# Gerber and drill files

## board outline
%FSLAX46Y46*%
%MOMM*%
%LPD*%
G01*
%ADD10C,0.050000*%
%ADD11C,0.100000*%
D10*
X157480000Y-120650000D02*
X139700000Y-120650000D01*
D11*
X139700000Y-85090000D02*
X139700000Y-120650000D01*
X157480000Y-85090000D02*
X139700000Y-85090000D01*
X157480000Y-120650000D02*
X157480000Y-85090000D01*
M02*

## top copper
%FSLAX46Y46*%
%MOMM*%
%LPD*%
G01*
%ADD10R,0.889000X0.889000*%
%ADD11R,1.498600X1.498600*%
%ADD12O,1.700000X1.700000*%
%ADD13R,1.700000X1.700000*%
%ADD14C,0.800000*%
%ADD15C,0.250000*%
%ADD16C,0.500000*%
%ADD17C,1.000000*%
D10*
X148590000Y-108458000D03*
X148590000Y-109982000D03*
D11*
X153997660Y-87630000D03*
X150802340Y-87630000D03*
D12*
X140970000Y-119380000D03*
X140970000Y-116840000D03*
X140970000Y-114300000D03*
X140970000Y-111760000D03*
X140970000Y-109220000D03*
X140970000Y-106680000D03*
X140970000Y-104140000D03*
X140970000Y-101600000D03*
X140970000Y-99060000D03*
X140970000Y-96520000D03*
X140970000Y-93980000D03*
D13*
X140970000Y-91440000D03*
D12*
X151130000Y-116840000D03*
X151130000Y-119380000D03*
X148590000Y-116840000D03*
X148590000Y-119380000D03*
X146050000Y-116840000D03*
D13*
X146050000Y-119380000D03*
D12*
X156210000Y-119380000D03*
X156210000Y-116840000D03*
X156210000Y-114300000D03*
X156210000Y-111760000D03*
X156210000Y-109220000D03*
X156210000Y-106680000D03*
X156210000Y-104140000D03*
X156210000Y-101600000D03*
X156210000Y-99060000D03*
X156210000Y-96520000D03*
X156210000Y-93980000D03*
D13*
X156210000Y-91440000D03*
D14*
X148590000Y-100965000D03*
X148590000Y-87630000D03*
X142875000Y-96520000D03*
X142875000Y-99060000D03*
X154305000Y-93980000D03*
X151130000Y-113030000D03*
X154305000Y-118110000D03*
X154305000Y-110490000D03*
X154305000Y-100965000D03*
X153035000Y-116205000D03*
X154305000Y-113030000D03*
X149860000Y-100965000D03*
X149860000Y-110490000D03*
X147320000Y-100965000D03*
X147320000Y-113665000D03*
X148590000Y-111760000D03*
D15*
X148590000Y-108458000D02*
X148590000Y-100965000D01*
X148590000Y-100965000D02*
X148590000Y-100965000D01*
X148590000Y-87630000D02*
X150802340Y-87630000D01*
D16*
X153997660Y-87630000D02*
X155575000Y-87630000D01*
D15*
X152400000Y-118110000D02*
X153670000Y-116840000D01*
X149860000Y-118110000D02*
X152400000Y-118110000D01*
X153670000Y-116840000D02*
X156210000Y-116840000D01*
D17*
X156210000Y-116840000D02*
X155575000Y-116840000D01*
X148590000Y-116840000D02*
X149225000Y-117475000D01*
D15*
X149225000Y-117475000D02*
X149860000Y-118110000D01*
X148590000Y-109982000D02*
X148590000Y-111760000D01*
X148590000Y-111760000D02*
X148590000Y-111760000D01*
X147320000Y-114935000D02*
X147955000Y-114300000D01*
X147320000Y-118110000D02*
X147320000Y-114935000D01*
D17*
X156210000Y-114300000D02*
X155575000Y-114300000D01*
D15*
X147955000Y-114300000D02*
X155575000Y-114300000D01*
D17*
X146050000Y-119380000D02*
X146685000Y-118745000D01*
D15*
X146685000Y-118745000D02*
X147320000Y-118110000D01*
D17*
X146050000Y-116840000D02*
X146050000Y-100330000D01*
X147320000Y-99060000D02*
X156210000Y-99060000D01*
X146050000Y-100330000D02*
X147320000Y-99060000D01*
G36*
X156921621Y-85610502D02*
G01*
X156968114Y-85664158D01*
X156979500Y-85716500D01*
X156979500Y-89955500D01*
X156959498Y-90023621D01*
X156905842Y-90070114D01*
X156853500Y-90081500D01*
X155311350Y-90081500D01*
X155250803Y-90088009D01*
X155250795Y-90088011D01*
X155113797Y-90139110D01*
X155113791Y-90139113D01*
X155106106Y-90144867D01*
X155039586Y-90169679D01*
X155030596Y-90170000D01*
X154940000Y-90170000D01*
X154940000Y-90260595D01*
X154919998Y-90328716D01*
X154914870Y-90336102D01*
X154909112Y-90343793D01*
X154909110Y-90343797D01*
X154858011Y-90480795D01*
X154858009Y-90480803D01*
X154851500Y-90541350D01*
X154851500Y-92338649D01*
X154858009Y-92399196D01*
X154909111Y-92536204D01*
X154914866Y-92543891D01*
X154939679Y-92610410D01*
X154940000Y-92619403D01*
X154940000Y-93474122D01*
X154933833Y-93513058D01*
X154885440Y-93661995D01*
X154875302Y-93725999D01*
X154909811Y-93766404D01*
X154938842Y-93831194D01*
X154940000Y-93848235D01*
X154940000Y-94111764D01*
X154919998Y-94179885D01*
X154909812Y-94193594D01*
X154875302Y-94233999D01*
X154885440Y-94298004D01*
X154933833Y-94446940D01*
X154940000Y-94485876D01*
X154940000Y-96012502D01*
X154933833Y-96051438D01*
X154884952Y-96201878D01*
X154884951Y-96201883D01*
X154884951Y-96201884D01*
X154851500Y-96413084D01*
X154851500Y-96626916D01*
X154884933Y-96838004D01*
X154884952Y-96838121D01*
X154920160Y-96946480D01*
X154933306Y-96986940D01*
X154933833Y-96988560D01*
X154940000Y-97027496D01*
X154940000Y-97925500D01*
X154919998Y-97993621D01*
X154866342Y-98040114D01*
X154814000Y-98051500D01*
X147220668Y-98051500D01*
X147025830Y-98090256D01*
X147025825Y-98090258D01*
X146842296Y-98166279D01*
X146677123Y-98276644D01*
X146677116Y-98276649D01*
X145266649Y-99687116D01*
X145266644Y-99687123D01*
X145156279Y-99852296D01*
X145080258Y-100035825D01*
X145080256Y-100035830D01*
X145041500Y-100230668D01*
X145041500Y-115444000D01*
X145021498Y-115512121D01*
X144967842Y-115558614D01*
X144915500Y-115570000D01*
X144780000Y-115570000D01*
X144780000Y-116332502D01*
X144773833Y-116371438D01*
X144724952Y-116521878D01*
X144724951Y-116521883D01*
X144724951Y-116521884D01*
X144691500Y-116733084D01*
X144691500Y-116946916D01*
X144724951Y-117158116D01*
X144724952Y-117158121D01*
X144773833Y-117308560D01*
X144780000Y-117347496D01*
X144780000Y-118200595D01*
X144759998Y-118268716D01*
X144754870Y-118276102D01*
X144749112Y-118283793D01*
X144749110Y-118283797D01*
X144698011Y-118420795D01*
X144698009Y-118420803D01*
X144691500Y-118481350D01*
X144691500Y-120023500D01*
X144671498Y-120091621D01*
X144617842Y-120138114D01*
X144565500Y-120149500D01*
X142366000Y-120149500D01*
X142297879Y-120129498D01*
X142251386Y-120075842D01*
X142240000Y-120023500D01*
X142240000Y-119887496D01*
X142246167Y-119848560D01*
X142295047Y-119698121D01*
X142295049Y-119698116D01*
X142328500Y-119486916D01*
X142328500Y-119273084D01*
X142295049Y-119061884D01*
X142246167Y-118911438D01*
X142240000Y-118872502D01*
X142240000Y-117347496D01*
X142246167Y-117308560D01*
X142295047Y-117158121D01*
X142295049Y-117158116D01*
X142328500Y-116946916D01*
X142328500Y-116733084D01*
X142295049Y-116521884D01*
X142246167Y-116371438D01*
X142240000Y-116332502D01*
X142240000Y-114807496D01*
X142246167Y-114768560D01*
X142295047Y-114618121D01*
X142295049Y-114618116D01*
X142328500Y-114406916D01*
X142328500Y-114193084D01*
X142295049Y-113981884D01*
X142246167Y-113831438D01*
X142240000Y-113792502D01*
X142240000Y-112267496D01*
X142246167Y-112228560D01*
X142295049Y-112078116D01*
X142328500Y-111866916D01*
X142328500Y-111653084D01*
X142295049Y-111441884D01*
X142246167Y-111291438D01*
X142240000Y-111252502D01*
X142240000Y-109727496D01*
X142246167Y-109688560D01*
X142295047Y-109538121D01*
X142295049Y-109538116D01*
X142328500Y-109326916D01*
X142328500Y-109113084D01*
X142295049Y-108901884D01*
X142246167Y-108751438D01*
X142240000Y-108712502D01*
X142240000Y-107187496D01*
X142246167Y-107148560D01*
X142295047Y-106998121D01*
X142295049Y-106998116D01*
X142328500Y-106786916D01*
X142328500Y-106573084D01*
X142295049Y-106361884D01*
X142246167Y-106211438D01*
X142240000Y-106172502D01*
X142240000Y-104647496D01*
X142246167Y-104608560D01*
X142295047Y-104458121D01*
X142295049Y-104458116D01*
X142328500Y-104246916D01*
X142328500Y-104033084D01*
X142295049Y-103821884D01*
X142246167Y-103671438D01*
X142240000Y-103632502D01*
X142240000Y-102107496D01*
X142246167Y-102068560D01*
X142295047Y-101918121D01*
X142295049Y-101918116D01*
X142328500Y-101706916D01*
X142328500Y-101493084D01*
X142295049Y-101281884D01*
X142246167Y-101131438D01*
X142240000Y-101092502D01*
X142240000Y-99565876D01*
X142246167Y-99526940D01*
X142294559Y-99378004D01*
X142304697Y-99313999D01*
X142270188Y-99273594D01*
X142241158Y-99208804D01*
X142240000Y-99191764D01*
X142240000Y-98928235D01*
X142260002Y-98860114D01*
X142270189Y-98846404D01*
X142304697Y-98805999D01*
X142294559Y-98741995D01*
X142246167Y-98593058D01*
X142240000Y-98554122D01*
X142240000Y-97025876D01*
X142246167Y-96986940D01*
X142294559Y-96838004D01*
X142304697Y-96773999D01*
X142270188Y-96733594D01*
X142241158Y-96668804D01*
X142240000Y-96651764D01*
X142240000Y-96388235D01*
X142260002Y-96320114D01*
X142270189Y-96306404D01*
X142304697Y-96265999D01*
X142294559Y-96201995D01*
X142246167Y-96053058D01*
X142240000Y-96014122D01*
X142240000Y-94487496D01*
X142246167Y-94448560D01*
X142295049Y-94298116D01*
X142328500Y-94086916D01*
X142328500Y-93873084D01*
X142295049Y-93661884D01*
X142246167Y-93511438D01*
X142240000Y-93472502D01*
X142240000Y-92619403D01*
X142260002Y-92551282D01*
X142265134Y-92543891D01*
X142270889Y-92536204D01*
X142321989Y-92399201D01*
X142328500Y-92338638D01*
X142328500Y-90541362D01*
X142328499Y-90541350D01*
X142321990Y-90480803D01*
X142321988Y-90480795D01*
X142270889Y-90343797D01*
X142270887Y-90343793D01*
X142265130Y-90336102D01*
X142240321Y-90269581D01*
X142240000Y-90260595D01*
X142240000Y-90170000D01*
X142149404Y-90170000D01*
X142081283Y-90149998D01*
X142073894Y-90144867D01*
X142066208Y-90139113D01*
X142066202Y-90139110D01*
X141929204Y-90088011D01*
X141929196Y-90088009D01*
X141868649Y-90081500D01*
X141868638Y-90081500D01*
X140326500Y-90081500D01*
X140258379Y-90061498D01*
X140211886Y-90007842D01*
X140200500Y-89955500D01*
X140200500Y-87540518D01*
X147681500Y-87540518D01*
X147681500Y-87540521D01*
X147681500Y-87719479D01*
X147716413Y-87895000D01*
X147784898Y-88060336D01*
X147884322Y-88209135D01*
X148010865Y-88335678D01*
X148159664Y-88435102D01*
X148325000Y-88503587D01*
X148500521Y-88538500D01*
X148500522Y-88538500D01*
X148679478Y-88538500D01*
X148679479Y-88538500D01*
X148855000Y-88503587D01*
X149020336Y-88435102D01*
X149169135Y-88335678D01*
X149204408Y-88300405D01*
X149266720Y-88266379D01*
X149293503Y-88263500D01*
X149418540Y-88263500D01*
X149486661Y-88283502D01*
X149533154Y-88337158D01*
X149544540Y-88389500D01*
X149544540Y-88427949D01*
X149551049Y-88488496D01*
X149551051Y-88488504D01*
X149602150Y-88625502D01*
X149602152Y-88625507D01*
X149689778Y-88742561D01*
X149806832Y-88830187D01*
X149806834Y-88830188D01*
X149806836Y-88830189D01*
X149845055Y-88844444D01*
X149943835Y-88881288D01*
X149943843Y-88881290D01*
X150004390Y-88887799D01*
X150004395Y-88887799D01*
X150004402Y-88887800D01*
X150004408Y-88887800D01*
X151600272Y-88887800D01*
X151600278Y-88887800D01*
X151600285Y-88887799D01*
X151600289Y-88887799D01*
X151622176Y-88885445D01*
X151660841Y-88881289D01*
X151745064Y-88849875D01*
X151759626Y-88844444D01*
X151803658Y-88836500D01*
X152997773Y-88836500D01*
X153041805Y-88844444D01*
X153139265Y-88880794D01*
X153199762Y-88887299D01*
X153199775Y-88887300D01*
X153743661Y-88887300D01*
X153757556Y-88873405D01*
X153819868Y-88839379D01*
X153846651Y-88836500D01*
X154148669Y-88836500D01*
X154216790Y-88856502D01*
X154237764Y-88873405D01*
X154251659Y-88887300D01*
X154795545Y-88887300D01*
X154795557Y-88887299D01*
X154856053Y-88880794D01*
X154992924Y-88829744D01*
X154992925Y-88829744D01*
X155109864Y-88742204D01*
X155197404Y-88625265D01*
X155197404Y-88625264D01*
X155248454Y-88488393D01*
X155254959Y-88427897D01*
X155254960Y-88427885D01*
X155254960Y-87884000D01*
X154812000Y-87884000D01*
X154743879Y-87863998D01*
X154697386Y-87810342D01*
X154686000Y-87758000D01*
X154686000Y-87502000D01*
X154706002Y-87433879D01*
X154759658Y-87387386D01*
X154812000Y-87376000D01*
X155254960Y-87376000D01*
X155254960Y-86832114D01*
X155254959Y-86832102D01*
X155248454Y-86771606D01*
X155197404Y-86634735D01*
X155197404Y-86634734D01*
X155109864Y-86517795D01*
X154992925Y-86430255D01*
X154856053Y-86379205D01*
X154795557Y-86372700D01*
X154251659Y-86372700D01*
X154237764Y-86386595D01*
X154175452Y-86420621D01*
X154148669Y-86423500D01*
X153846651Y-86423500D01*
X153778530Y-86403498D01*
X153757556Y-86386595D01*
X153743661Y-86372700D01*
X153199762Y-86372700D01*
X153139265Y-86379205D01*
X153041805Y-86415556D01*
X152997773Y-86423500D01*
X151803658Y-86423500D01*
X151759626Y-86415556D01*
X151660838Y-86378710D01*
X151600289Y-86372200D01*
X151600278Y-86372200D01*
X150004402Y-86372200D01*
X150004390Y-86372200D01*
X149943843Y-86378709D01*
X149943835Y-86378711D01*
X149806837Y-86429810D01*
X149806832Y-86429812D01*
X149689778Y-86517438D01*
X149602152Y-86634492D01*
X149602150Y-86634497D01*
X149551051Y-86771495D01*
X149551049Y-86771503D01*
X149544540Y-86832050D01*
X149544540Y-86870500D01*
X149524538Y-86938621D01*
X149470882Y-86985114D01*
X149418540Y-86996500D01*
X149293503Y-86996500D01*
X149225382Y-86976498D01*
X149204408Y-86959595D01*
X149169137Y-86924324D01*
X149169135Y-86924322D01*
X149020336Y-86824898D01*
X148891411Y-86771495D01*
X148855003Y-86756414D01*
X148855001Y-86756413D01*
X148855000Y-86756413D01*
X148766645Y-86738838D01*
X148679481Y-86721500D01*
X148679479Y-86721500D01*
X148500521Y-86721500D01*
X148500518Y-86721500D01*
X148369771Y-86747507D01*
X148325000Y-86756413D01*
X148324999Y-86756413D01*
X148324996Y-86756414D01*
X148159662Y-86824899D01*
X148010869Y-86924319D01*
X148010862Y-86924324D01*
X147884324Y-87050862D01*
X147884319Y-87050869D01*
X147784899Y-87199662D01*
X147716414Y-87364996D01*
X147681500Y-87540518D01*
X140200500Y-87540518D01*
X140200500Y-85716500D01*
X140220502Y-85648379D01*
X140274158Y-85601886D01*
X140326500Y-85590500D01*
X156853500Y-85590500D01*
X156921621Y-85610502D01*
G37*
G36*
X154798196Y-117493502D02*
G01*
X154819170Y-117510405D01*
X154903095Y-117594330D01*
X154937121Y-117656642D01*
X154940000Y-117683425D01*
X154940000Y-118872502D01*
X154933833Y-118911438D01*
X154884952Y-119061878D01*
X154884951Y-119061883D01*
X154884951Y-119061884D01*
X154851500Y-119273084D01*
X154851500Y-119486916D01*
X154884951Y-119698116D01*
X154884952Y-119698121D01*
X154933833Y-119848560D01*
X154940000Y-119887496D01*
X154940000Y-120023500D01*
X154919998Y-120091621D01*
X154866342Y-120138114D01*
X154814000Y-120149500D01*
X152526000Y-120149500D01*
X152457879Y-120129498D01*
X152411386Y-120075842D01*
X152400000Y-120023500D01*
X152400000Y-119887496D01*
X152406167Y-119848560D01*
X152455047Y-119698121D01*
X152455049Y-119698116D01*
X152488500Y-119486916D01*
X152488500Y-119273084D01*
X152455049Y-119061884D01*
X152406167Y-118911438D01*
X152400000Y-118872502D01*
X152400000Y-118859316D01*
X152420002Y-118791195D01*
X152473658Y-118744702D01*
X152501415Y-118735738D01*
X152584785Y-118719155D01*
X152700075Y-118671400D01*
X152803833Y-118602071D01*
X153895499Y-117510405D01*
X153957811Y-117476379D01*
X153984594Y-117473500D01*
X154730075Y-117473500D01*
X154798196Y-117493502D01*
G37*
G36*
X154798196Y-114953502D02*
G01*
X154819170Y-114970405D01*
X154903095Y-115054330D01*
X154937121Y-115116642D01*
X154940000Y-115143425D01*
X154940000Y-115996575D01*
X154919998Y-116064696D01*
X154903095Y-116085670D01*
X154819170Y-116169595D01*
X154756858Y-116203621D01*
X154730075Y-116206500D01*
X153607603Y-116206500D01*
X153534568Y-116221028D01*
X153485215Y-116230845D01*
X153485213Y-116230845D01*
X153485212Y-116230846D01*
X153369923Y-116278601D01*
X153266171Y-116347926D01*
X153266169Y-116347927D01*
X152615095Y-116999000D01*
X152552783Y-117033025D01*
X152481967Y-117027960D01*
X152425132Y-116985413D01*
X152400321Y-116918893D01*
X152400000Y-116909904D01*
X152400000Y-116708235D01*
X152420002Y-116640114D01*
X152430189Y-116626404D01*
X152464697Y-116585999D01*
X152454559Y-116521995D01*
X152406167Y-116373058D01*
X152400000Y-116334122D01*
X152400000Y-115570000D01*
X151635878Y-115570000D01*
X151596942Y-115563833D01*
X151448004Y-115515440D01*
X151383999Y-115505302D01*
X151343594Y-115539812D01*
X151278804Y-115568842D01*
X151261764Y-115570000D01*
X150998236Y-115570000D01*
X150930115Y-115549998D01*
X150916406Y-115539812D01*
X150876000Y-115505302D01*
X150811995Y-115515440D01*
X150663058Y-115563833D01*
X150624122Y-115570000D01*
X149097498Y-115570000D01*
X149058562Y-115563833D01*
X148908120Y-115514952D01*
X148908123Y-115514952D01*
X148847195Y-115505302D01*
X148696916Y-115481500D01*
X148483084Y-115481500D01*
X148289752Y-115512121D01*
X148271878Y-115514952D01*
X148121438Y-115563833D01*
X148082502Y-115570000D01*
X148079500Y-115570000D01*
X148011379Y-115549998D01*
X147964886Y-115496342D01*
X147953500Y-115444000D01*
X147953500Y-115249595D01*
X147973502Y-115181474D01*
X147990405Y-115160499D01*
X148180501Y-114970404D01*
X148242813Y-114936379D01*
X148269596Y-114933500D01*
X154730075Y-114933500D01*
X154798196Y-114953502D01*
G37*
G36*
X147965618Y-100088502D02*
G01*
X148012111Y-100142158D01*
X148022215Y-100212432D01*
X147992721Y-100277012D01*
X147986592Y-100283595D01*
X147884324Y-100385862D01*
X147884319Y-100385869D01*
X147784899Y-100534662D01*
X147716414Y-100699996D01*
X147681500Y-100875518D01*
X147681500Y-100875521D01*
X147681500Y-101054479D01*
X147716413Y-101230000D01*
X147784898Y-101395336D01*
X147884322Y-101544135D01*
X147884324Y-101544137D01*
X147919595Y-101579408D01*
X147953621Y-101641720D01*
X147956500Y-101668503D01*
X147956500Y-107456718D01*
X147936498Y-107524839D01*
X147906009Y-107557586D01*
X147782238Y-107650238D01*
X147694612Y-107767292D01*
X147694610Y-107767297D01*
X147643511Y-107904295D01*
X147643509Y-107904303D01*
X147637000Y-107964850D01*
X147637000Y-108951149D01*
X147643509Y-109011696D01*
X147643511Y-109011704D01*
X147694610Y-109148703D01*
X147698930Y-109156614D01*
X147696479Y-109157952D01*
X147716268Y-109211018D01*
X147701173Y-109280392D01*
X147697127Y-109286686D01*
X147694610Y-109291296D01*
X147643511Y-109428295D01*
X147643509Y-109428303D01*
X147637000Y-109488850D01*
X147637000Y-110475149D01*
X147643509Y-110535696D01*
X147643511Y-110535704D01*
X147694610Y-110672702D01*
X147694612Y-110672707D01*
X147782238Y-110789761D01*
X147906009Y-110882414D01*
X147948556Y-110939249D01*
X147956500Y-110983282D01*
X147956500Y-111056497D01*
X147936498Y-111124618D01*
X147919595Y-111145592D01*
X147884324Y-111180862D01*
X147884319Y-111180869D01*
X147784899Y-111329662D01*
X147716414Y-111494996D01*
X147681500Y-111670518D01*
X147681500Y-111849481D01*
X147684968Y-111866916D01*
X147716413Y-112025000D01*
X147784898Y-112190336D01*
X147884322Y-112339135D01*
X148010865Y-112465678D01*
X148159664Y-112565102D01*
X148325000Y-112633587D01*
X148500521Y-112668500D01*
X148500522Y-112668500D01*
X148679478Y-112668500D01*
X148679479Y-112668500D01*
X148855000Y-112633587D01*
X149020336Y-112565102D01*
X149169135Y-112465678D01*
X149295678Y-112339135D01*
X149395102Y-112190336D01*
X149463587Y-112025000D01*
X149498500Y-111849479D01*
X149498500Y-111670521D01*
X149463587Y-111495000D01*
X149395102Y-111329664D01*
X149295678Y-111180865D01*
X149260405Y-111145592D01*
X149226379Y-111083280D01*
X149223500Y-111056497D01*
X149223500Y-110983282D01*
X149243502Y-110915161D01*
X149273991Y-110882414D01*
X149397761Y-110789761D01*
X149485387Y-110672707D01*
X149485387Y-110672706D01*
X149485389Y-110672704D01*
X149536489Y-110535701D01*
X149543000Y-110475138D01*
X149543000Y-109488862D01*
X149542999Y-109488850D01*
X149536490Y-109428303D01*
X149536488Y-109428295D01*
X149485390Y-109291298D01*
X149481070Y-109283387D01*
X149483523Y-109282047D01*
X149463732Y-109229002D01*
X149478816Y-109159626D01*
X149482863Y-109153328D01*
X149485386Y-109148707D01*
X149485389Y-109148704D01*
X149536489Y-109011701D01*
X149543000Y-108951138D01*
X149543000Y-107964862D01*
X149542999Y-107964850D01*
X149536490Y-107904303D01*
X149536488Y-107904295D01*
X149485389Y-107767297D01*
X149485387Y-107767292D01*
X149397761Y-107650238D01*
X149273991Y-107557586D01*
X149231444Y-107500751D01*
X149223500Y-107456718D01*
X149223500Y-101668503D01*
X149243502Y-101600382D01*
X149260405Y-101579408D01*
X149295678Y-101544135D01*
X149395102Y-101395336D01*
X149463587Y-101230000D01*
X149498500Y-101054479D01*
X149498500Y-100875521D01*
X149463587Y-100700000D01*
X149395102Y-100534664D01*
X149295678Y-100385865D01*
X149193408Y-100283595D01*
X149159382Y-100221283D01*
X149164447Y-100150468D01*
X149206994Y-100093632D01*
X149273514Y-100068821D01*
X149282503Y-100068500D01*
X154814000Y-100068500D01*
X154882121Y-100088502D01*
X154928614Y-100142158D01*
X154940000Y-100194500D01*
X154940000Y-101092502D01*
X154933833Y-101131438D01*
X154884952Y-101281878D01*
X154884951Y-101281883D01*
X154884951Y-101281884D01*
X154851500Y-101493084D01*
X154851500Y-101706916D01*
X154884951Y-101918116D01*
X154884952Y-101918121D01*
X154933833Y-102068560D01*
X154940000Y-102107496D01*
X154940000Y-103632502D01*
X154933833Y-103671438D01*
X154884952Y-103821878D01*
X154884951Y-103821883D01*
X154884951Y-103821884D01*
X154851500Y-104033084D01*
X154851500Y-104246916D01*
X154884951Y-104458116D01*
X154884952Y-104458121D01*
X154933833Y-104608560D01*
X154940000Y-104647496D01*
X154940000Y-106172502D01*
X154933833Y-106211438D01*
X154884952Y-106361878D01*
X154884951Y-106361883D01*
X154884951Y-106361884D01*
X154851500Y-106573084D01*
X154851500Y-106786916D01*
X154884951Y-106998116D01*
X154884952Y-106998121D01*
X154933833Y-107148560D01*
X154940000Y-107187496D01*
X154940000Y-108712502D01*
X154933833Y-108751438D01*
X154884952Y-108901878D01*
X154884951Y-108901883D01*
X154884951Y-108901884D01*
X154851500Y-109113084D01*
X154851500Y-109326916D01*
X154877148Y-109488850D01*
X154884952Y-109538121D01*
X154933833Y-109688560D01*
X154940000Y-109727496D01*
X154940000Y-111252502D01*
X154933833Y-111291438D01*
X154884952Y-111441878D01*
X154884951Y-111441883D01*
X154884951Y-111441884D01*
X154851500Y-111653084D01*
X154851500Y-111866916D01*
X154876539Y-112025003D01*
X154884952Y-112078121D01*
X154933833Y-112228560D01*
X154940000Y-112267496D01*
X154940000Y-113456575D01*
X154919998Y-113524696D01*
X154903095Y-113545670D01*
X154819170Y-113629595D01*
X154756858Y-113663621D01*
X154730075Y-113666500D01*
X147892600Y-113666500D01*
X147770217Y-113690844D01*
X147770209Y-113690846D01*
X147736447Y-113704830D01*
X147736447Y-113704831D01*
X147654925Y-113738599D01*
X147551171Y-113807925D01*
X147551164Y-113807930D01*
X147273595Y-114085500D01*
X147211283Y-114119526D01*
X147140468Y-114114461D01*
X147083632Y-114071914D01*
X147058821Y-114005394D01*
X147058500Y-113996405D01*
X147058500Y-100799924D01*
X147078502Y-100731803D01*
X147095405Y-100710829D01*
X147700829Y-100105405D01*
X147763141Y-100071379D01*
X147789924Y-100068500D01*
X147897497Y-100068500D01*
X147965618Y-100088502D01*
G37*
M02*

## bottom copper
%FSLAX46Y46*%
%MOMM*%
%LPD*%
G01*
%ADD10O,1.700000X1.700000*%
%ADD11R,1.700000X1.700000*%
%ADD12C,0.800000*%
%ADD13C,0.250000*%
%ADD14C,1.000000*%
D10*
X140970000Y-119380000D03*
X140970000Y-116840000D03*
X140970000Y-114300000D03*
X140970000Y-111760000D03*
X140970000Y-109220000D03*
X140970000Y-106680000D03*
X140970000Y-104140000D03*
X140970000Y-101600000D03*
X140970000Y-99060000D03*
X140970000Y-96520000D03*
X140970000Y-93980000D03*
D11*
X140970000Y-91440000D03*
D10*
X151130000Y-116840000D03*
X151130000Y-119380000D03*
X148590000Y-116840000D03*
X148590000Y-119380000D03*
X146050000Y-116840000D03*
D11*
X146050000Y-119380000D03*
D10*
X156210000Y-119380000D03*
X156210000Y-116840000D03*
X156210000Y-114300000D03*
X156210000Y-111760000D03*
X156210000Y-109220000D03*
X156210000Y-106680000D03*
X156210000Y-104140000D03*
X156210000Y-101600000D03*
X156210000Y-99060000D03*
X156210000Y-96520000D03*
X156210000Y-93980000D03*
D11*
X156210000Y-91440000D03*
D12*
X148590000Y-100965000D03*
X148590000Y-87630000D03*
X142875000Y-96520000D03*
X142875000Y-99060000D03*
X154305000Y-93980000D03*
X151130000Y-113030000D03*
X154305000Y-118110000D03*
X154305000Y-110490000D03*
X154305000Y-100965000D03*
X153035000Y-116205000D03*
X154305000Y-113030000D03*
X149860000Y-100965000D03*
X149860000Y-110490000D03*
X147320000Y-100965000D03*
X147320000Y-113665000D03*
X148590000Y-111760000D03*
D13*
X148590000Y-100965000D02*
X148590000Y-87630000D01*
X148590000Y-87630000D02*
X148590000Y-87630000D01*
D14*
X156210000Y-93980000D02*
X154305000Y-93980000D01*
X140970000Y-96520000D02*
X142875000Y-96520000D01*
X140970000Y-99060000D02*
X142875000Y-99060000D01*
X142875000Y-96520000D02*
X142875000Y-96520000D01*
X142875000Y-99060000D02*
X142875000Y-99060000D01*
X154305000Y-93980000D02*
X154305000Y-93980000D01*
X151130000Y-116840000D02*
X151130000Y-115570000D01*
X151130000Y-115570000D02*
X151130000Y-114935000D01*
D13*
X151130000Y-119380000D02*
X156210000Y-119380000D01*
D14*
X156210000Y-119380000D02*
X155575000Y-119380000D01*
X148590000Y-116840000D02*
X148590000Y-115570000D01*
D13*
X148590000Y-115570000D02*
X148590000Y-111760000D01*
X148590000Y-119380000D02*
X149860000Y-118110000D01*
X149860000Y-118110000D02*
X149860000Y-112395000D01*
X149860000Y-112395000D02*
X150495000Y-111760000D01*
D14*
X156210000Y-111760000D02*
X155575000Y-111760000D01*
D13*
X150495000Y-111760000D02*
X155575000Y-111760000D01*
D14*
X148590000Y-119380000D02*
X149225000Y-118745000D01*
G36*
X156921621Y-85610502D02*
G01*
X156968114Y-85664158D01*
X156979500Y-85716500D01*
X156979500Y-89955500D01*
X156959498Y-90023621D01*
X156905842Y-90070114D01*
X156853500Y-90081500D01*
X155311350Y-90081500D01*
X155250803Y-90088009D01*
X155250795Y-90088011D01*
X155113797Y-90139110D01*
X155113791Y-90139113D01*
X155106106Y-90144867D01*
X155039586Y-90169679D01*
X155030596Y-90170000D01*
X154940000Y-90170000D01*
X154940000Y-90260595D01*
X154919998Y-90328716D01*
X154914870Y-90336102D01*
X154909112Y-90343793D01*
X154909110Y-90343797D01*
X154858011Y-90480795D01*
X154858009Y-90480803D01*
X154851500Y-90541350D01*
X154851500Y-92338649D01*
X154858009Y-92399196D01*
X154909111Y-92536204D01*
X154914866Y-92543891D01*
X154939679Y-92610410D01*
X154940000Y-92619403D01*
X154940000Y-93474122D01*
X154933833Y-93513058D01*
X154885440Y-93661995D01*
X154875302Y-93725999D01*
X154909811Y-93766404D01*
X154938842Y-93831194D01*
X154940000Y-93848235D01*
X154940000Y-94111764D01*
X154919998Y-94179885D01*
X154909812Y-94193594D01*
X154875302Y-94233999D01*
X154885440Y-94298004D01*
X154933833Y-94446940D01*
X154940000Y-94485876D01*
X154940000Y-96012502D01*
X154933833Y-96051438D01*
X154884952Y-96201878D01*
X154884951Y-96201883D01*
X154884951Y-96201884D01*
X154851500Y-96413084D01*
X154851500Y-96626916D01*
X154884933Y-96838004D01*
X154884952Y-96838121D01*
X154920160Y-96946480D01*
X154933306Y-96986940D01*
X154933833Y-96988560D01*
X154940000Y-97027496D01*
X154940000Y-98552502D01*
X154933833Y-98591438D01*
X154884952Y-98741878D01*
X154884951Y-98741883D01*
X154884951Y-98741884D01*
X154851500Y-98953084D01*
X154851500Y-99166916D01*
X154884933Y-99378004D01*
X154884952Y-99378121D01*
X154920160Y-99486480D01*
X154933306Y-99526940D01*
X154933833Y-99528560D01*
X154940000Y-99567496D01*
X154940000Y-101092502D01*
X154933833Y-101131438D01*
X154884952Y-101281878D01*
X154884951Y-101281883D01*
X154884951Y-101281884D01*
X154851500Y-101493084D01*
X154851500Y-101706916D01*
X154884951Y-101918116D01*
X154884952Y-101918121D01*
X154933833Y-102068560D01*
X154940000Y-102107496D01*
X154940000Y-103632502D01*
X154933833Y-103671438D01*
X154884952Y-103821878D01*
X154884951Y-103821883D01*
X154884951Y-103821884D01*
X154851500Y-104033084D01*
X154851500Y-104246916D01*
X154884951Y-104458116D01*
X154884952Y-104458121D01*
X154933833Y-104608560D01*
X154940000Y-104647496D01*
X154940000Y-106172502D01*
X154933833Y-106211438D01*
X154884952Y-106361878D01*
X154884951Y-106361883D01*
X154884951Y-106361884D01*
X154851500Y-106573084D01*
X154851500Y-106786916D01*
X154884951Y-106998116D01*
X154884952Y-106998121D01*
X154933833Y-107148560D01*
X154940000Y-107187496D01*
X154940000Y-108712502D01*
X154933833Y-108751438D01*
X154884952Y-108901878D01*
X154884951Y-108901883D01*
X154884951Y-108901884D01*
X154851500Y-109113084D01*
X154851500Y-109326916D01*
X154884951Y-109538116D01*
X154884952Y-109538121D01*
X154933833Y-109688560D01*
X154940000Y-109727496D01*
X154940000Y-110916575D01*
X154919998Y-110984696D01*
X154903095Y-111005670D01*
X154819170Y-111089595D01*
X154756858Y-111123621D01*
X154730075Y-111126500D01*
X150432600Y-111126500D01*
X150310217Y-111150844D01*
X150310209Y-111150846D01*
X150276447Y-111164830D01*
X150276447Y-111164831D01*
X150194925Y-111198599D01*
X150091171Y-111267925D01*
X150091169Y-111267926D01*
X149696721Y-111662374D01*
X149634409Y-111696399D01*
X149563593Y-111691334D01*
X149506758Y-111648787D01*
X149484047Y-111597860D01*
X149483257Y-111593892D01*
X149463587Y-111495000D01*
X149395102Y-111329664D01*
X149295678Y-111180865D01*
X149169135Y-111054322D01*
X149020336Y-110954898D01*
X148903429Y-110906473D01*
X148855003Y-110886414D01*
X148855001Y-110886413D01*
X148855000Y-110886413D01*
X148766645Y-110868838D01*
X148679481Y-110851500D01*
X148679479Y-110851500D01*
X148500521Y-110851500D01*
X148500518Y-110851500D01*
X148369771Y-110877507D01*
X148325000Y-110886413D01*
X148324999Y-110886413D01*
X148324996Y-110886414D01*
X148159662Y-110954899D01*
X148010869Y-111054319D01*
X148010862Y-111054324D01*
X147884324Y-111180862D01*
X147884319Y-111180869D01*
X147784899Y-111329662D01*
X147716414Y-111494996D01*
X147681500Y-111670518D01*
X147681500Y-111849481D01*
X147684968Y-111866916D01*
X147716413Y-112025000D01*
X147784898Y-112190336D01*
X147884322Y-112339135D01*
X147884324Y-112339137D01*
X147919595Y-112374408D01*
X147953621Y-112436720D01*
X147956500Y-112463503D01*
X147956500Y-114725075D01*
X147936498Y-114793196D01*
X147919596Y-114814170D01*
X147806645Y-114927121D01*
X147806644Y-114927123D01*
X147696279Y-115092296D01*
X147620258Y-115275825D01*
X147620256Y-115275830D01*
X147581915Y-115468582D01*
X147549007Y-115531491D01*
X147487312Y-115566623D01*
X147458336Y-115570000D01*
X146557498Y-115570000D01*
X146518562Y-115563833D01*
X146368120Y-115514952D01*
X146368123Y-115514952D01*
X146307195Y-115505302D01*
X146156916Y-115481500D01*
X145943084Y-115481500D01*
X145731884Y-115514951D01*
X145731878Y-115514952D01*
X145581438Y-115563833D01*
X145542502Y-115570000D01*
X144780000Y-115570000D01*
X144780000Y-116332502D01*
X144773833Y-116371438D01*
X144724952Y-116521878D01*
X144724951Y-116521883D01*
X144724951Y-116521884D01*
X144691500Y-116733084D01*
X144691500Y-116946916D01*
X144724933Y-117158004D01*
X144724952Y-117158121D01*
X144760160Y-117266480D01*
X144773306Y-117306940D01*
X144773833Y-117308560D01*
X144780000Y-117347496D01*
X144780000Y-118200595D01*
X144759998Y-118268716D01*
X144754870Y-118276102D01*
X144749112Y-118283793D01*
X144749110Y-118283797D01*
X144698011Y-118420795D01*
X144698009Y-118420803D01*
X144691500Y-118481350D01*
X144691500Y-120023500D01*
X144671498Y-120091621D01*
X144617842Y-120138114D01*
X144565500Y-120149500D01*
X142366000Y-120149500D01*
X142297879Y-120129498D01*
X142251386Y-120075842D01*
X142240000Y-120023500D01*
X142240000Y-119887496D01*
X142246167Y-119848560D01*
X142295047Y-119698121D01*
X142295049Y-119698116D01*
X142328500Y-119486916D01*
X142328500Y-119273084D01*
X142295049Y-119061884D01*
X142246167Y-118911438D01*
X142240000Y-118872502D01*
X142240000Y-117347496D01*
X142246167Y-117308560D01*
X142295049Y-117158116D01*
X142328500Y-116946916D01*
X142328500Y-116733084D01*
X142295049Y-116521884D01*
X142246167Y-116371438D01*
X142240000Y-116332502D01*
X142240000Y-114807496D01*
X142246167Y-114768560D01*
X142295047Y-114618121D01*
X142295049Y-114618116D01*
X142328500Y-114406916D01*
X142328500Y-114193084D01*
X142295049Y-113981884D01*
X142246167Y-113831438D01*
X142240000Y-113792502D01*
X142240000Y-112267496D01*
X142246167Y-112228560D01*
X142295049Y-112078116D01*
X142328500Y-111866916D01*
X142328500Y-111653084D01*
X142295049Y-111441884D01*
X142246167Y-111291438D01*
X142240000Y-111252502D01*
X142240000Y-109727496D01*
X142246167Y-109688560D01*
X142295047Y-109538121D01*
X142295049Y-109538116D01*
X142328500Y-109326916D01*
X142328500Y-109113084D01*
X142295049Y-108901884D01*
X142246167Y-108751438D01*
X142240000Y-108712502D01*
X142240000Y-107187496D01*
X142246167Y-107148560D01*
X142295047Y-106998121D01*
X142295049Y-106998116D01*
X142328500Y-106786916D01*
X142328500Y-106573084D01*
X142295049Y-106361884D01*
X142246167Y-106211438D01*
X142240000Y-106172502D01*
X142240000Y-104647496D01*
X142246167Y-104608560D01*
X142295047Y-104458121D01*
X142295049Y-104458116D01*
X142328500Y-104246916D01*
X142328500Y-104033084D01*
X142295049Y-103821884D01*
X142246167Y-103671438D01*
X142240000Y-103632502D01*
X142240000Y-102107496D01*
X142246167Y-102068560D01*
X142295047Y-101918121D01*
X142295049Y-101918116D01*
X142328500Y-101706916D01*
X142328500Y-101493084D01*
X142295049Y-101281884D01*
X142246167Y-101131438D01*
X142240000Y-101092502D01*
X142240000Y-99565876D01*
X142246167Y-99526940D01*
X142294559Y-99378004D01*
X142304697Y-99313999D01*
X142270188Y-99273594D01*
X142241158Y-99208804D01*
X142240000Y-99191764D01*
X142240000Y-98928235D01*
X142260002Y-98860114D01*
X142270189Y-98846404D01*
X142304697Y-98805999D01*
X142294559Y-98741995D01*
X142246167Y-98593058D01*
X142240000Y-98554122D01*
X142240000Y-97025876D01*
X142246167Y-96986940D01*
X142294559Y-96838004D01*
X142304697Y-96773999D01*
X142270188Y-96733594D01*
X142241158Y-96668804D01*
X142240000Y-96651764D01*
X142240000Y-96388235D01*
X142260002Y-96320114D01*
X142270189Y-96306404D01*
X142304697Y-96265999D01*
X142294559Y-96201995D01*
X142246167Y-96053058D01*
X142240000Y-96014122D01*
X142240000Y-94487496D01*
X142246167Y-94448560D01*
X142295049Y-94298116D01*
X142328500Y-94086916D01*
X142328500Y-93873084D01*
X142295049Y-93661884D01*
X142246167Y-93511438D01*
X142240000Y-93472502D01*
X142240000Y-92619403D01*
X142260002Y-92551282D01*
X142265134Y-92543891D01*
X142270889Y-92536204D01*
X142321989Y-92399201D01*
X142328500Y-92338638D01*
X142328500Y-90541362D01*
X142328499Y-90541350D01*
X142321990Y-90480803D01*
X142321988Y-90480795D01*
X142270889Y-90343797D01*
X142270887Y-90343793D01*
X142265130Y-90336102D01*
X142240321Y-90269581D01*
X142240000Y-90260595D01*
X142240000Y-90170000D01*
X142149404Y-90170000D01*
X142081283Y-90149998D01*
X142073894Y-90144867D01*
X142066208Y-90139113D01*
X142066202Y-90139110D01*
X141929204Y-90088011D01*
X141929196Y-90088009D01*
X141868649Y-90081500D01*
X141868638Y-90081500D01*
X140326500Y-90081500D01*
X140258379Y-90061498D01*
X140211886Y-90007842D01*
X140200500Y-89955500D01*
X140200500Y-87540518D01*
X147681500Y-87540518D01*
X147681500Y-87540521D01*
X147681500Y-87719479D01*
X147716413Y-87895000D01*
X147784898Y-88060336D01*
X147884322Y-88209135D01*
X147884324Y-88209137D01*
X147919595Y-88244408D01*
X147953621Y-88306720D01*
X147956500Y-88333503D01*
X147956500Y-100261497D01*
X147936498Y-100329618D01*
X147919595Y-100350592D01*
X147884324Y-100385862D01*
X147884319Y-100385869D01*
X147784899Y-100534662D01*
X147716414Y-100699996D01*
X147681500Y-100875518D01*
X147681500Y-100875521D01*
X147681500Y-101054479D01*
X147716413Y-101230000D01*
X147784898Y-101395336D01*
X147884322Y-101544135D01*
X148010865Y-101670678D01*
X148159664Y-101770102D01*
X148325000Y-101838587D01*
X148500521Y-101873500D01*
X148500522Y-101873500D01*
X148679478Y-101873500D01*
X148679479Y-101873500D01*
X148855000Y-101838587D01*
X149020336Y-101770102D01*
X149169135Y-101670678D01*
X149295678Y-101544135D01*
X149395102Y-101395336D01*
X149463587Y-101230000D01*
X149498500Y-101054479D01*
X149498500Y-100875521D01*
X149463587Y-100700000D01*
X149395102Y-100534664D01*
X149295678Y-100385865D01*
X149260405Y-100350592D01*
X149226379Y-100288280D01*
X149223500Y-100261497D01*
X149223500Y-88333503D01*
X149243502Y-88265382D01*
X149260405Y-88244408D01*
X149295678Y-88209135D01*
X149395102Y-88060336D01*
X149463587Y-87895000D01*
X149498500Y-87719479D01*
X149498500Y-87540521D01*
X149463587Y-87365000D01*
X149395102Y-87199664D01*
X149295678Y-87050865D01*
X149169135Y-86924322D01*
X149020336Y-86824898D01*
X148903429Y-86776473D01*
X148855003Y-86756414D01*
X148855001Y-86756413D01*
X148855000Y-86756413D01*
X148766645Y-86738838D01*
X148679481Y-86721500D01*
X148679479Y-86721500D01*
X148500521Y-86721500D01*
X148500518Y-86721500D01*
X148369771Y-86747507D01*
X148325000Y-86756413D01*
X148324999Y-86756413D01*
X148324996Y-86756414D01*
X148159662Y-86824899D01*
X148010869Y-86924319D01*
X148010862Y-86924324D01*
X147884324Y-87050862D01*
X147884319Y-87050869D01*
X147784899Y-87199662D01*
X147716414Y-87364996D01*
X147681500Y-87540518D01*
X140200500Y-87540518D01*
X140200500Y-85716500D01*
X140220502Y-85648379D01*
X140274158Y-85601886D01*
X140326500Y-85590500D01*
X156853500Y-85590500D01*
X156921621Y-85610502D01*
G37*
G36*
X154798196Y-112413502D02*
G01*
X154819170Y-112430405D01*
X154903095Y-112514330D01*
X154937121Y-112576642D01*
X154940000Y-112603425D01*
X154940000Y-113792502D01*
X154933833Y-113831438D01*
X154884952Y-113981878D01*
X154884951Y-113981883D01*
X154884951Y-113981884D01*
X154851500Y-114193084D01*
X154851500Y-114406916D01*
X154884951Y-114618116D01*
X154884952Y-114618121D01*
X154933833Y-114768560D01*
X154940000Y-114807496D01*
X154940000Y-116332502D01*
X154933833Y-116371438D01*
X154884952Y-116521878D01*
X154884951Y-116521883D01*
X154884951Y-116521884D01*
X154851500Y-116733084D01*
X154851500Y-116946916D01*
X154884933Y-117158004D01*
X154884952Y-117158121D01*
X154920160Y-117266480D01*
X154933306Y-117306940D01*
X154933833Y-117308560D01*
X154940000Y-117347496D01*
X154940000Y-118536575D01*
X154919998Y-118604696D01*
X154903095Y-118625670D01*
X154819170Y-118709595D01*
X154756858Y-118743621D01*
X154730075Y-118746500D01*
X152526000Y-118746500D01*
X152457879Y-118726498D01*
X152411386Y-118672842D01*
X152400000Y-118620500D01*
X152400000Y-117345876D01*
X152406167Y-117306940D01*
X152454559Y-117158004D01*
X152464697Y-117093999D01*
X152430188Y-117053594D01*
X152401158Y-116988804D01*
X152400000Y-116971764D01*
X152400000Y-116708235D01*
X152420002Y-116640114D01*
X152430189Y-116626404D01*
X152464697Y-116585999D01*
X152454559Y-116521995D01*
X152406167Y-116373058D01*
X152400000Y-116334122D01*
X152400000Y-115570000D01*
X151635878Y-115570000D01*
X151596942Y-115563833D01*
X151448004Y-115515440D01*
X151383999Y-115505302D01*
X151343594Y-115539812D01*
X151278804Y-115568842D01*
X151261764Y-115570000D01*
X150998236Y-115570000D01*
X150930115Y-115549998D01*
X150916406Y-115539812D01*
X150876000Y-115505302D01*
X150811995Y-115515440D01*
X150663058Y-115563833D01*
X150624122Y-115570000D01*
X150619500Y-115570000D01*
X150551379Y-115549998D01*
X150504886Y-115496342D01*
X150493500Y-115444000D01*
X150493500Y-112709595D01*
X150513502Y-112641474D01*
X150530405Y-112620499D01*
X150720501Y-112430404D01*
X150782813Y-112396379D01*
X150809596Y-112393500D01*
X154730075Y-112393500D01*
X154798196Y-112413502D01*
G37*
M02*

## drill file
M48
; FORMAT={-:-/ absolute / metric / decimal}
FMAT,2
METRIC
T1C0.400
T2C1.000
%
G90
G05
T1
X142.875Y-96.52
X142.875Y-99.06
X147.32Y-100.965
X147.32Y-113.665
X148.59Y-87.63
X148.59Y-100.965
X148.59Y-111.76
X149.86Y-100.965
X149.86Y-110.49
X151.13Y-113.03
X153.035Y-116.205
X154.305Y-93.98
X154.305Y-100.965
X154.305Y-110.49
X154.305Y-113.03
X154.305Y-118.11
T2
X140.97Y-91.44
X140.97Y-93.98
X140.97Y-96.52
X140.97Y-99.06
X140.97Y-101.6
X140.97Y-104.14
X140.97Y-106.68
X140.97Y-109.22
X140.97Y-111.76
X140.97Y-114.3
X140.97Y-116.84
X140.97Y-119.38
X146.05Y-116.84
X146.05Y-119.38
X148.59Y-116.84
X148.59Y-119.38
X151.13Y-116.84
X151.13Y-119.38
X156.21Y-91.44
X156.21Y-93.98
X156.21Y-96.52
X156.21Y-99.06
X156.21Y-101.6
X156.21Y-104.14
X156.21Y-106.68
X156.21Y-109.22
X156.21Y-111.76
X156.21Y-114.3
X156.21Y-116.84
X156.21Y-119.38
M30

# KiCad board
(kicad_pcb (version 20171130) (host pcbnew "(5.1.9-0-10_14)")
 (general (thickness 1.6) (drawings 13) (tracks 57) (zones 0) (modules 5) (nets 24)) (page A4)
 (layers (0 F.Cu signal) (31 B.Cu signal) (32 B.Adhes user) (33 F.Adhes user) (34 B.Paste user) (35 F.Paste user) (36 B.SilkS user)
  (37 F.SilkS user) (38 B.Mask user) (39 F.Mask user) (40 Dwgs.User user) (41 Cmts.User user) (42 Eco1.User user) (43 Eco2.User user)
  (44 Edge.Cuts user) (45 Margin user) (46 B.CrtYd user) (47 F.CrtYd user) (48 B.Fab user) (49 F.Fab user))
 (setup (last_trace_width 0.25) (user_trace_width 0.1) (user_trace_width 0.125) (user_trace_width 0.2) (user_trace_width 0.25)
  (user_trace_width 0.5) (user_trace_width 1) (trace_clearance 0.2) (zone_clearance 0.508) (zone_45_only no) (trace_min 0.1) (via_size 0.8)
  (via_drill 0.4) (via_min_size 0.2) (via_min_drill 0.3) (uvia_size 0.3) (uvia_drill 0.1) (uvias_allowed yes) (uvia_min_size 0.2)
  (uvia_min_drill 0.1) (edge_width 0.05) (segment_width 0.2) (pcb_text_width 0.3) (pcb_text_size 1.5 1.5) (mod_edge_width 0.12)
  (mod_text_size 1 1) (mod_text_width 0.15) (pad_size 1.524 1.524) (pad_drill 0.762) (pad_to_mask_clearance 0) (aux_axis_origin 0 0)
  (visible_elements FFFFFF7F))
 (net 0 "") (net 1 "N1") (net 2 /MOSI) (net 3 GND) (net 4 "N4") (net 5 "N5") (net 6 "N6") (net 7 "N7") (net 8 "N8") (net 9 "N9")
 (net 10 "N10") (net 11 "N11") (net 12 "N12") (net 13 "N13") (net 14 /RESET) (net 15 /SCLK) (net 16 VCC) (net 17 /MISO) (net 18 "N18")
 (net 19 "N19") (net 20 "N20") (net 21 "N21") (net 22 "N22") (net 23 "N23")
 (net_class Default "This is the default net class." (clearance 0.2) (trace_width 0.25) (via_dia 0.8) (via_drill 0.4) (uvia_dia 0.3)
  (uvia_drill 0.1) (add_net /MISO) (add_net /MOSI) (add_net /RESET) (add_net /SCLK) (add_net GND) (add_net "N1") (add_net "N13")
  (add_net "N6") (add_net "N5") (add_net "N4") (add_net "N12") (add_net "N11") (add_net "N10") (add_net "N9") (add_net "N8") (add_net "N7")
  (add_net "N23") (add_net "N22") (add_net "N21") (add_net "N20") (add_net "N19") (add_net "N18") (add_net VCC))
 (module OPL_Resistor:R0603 (layer F.Cu) (at 148.59 109.22 90)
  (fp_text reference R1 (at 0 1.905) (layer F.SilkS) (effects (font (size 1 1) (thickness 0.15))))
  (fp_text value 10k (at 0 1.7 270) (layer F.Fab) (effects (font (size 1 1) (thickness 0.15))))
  (pad 2 smd rect (at 0.762 0 90) (size 0.889 0.889) (layers F.Cu F.Paste F.Mask) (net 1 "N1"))
  (pad 1 smd rect (at -0.762 0 90) (size 0.889 0.889) (layers F.Cu F.Paste F.Mask) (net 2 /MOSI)))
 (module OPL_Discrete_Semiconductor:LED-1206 (layer F.Cu) (at 152.4 87.63 180)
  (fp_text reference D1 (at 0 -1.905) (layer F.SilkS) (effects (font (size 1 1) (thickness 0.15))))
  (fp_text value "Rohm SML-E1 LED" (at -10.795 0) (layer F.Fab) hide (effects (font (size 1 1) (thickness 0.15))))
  (pad 1 smd rect (at -1.59766 0 180) (size 1.4986 1.4986) (layers F.Cu F.Paste F.Mask) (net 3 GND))
  (pad 2 smd rect (at 1.59766 0 180) (size 1.4986 1.4986) (layers F.Cu F.Paste F.Mask) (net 1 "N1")))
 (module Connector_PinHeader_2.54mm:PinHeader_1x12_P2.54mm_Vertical (layer F.Cu) (at 140.97 91.44)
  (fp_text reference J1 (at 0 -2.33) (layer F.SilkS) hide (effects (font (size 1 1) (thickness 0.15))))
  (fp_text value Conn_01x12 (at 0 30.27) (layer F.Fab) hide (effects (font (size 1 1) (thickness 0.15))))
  (pad 12 thru_hole oval (at 0 27.94) (size 1.7 1.7) (drill 1) (layers *.Cu *.Mask) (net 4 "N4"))
  (pad 11 thru_hole oval (at 0 25.4) (size 1.7 1.7) (drill 1) (layers *.Cu *.Mask) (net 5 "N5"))
  (pad 10 thru_hole oval (at 0 22.86) (size 1.7 1.7) (drill 1) (layers *.Cu *.Mask) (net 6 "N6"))
  (pad 9 thru_hole oval (at 0 20.32) (size 1.7 1.7) (drill 1) (layers *.Cu *.Mask) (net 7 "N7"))
  (pad 8 thru_hole oval (at 0 17.78) (size 1.7 1.7) (drill 1) (layers *.Cu *.Mask) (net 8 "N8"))
  (pad 7 thru_hole oval (at 0 15.24) (size 1.7 1.7) (drill 1) (layers *.Cu *.Mask) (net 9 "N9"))
  (pad 6 thru_hole oval (at 0 12.7) (size 1.7 1.7) (drill 1) (layers *.Cu *.Mask) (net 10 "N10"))
  (pad 5 thru_hole oval (at 0 10.16) (size 1.7 1.7) (drill 1) (layers *.Cu *.Mask) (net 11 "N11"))
  (pad 4 thru_hole oval (at 0 7.62) (size 1.7 1.7) (drill 1) (layers *.Cu *.Mask) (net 3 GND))
  (pad 3 thru_hole oval (at 0 5.08) (size 1.7 1.7) (drill 1) (layers *.Cu *.Mask) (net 3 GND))
  (pad 2 thru_hole oval (at 0 2.54) (size 1.7 1.7) (drill 1) (layers *.Cu *.Mask) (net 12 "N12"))
  (pad 1 thru_hole rect (at 0 0) (size 1.7 1.7) (drill 1) (layers *.Cu *.Mask) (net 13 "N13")))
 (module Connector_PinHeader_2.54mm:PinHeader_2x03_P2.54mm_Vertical (layer F.Cu) (at 146.05 119.38 90)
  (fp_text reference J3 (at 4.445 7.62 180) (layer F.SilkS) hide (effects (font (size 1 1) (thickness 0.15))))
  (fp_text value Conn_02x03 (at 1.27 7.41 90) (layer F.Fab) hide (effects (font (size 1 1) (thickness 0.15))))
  (pad 6 thru_hole oval (at 2.54 5.08 90) (size 1.7 1.7) (drill 1) (layers *.Cu *.Mask) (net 3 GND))
  (pad 5 thru_hole oval (at 0 5.08 90) (size 1.7 1.7) (drill 1) (layers *.Cu *.Mask) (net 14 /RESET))
  (pad 4 thru_hole oval (at 2.54 2.54 90) (size 1.7 1.7) (drill 1) (layers *.Cu *.Mask) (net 2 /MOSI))
  (pad 3 thru_hole oval (at 0 2.54 90) (size 1.7 1.7) (drill 1) (layers *.Cu *.Mask) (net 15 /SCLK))
  (pad 2 thru_hole oval (at 2.54 0 90) (size 1.7 1.7) (drill 1) (layers *.Cu *.Mask) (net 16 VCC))
  (pad 1 thru_hole rect (at 0 0 90) (size 1.7 1.7) (drill 1) (layers *.Cu *.Mask) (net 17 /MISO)))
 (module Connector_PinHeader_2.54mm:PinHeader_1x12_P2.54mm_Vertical (layer F.Cu) (at 156.21 91.44)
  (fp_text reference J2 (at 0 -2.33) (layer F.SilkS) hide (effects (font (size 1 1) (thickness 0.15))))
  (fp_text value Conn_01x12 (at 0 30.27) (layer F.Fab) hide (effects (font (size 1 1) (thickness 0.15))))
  (pad 12 thru_hole oval (at 0 27.94) (size 1.7 1.7) (drill 1) (layers *.Cu *.Mask) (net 14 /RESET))
  (pad 11 thru_hole oval (at 0 25.4) (size 1.7 1.7) (drill 1) (layers *.Cu *.Mask) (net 2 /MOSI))
  (pad 10 thru_hole oval (at 0 22.86) (size 1.7 1.7) (drill 1) (layers *.Cu *.Mask) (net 17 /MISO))
  (pad 9 thru_hole oval (at 0 20.32) (size 1.7 1.7) (drill 1) (layers *.Cu *.Mask) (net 15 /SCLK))
  (pad 8 thru_hole oval (at 0 17.78) (size 1.7 1.7) (drill 1) (layers *.Cu *.Mask) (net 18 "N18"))
  (pad 7 thru_hole oval (at 0 15.24) (size 1.7 1.7) (drill 1) (layers *.Cu *.Mask) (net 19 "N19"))
  (pad 6 thru_hole oval (at 0 12.7) (size 1.7 1.7) (drill 1) (layers *.Cu *.Mask) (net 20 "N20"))
  (pad 5 thru_hole oval (at 0 10.16) (size 1.7 1.7) (drill 1) (layers *.Cu *.Mask) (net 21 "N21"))
  (pad 4 thru_hole oval (at 0 7.62) (size 1.7 1.7) (drill 1) (layers *.Cu *.Mask) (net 16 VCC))
  (pad 3 thru_hole oval (at 0 5.08) (size 1.7 1.7) (drill 1) (layers *.Cu *.Mask) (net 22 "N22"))
  (pad 2 thru_hole oval (at 0 2.54) (size 1.7 1.7) (drill 1) (layers *.Cu *.Mask) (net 3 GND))
  (pad 1 thru_hole rect (at 0 0) (size 1.7 1.7) (drill 1) (layers *.Cu *.Mask) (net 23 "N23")))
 (gr_line (start 157.48 120.65) (end 139.7 120.65) (layer Edge.Cuts) (width 0.05))
 (gr_line (start 139.7 85.09) (end 139.7 120.65) (layer Edge.Cuts) (width 0.1))
 (gr_line (start 157.48 85.09) (end 139.7 85.09) (layer Edge.Cuts) (width 0.1))
 (gr_line (start 157.48 120.65) (end 157.48 85.09) (layer Edge.Cuts) (width 0.1))
 (segment (start 148.59 108.458) (end 148.59 100.965) (width 0.25) (layer F.Cu) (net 1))
 (segment (start 148.59 100.965) (end 148.59 100.965) (width 0.25) (layer F.Cu) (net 1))
 (via (at 148.59 100.965) (size 0.8) (drill 0.4) (layers F.Cu B.Cu) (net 1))
 (segment (start 148.59 100.965) (end 148.59 87.63) (width 0.25) (layer B.Cu) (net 1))
 (segment (start 148.59 87.63) (end 148.59 87.63) (width 0.25) (layer B.Cu) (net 1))
 (via (at 148.59 87.63) (size 0.8) (drill 0.4) (layers F.Cu B.Cu) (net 1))
 (segment (start 148.59 87.63) (end 150.80234 87.63) (width 0.25) (layer F.Cu) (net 1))
 (segment (start 156.21 93.98) (end 154.305 93.98) (width 1) (layer B.Cu) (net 3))
 (segment (start 140.97 96.52) (end 142.875 96.52) (width 1) (layer B.Cu) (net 3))
 (segment (start 140.97 99.06) (end 142.875 99.06) (width 1) (layer B.Cu) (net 3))
 (segment (start 142.875 96.52) (end 142.875 96.52) (width 1) (layer B.Cu) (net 3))
 (via (at 142.875 96.52) (size 0.8) (drill 0.4) (layers F.Cu B.Cu) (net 3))
 (segment (start 142.875 99.06) (end 142.875 99.06) (width 1) (layer B.Cu) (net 3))
 (via (at 142.875 99.06) (size 0.8) (drill 0.4) (layers F.Cu B.Cu) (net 3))
 (segment (start 154.305 93.98) (end 154.305 93.98) (width 1) (layer B.Cu) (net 3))
 (via (at 154.305 93.98) (size 0.8) (drill 0.4) (layers F.Cu B.Cu) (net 3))
 (via (at 151.13 113.03) (size 0.8) (drill 0.4) (layers F.Cu B.Cu) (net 3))
 (via (at 154.305 118.11) (size 0.8) (drill 0.4) (layers F.Cu B.Cu) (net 3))
 (segment (start 151.13 116.84) (end 151.13 115.57) (width 1) (layer B.Cu) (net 3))
 (via (at 154.305 110.49) (size 0.8) (drill 0.4) (layers F.Cu B.Cu) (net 3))
 (via (at 154.305 100.965) (size 0.8) (drill 0.4) (layers F.Cu B.Cu) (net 3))
 (segment (start 151.13 115.57) (end 151.13 114.935) (width 1) (layer B.Cu) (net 3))
 (via (at 153.035 116.205) (size 0.8) (drill 0.4) (layers F.Cu B.Cu) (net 3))
 (via (at 154.305 113.03) (size 0.8) (drill 0.4) (layers F.Cu B.Cu) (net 3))
 (via (at 149.86 100.965) (size 0.8) (drill 0.4) (layers F.Cu B.Cu) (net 3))
 (via (at 149.86 110.49) (size 0.8) (drill 0.4) (layers F.Cu B.Cu) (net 3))
 (via (at 147.32 100.965) (size 0.8) (drill 0.4) (layers F.Cu B.Cu) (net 3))
 (via (at 147.32 113.665) (size 0.8) (drill 0.4) (layers F.Cu B.Cu) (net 3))
 (segment (start 153.99766 87.63) (end 155.575 87.63) (width 0.5) (layer F.Cu) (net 3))
 (segment (start 151.13 119.38) (end 156.21 119.38) (width 0.25) (layer B.Cu) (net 14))
 (segment (start 156.21 119.38) (end 155.575 119.38) (width 1) (layer B.Cu) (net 14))
 (segment (start 152.4 118.11) (end 153.67 116.84) (width 0.25) (layer F.Cu) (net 2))
 (segment (start 149.86 118.11) (end 152.4 118.11) (width 0.25) (layer F.Cu) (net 2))
 (segment (start 153.67 116.84) (end 156.21 116.84) (width 0.25) (layer F.Cu) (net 2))
 (segment (start 156.21 116.84) (end 155.575 116.84) (width 1) (layer F.Cu) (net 2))
 (segment (start 148.59 116.84) (end 149.225 117.475) (width 1) (layer F.Cu) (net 2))
 (segment (start 149.225 117.475) (end 149.86 118.11) (width 0.25) (layer F.Cu) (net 2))
 (segment (start 148.59 116.84) (end 148.59 115.57) (width 1) (layer B.Cu) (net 2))
 (segment (start 148.59 109.982) (end 148.59 111.76) (width 0.25) (layer F.Cu) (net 2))
 (segment (start 148.59 111.76) (end 148.59 111.76) (width 0.25) (layer F.Cu) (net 2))
 (via (at 148.59 111.76) (size 0.8) (drill 0.4) (layers F.Cu B.Cu) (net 2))
 (segment (start 148.59 115.57) (end 148.59 111.76) (width 0.25) (layer B.Cu) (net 2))
 (segment (start 147.32 114.935) (end 147.955 114.3) (width 0.25) (layer F.Cu) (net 17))
 (segment (start 147.32 118.11) (end 147.32 114.935) (width 0.25) (layer F.Cu) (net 17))
 (segment (start 156.21 114.3) (end 155.575 114.3) (width 1) (layer F.Cu) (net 17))
 (segment (start 147.955 114.3) (end 155.575 114.3) (width 0.25) (layer F.Cu) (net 17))
 (segment (start 146.05 119.38) (end 146.685 118.745) (width 1) (layer F.Cu) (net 17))
 (segment (start 146.685 118.745) (end 147.32 118.11) (width 0.25) (layer F.Cu) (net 17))
 (segment (start 148.59 119.38) (end 149.86 118.11) (width 0.25) (layer B.Cu) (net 15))
 (segment (start 149.86 118.11) (end 149.86 112.395) (width 0.25) (layer B.Cu) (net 15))
 (segment (start 149.86 112.395) (end 150.495 111.76) (width 0.25) (layer B.Cu) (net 15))
 (segment (start 156.21 111.76) (end 155.575 111.76) (width 1) (layer B.Cu) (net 15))
 (segment (start 150.495 111.76) (end 155.575 111.76) (width 0.25) (layer B.Cu) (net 15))
 (segment (start 148.59 119.38) (end 149.225 118.745) (width 1) (layer B.Cu) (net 15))
 (segment (start 146.05 116.84) (end 146.05 100.33) (width 1) (layer F.Cu) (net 16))
 (segment (start 147.32 99.06) (end 156.21 99.06) (width 1) (layer F.Cu) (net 16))
 (segment (start 146.05 100.33) (end 147.32 99.06) (width 1) (layer F.Cu) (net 16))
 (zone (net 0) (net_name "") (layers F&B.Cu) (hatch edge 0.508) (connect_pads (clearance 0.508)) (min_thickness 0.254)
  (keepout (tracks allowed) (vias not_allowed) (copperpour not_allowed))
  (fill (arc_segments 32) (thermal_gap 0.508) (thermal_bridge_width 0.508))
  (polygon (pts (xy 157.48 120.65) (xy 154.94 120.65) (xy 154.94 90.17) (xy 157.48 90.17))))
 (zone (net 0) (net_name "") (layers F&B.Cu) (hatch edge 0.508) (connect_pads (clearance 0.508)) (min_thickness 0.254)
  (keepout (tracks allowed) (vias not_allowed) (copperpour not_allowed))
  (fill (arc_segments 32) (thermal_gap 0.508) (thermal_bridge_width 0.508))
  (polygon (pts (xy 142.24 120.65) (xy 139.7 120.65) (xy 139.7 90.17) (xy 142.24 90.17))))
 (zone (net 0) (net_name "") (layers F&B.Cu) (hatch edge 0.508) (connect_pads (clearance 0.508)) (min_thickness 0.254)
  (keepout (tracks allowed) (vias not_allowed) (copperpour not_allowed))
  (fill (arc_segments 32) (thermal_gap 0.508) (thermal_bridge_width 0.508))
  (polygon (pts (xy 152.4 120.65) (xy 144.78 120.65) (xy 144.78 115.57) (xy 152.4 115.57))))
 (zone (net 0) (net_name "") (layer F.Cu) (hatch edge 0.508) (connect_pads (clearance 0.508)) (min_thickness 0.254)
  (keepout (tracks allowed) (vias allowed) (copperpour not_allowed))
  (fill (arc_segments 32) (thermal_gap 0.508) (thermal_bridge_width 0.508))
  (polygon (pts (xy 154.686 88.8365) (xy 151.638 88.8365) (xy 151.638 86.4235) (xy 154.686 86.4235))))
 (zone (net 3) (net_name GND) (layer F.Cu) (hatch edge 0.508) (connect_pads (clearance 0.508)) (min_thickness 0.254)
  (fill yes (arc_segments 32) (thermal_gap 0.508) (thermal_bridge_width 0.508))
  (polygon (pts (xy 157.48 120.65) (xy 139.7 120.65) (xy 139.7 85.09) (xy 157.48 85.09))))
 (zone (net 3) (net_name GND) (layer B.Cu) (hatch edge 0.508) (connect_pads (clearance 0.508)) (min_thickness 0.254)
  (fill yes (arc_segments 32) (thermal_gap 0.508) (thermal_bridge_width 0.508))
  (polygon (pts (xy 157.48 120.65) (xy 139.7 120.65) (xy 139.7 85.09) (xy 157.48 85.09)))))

